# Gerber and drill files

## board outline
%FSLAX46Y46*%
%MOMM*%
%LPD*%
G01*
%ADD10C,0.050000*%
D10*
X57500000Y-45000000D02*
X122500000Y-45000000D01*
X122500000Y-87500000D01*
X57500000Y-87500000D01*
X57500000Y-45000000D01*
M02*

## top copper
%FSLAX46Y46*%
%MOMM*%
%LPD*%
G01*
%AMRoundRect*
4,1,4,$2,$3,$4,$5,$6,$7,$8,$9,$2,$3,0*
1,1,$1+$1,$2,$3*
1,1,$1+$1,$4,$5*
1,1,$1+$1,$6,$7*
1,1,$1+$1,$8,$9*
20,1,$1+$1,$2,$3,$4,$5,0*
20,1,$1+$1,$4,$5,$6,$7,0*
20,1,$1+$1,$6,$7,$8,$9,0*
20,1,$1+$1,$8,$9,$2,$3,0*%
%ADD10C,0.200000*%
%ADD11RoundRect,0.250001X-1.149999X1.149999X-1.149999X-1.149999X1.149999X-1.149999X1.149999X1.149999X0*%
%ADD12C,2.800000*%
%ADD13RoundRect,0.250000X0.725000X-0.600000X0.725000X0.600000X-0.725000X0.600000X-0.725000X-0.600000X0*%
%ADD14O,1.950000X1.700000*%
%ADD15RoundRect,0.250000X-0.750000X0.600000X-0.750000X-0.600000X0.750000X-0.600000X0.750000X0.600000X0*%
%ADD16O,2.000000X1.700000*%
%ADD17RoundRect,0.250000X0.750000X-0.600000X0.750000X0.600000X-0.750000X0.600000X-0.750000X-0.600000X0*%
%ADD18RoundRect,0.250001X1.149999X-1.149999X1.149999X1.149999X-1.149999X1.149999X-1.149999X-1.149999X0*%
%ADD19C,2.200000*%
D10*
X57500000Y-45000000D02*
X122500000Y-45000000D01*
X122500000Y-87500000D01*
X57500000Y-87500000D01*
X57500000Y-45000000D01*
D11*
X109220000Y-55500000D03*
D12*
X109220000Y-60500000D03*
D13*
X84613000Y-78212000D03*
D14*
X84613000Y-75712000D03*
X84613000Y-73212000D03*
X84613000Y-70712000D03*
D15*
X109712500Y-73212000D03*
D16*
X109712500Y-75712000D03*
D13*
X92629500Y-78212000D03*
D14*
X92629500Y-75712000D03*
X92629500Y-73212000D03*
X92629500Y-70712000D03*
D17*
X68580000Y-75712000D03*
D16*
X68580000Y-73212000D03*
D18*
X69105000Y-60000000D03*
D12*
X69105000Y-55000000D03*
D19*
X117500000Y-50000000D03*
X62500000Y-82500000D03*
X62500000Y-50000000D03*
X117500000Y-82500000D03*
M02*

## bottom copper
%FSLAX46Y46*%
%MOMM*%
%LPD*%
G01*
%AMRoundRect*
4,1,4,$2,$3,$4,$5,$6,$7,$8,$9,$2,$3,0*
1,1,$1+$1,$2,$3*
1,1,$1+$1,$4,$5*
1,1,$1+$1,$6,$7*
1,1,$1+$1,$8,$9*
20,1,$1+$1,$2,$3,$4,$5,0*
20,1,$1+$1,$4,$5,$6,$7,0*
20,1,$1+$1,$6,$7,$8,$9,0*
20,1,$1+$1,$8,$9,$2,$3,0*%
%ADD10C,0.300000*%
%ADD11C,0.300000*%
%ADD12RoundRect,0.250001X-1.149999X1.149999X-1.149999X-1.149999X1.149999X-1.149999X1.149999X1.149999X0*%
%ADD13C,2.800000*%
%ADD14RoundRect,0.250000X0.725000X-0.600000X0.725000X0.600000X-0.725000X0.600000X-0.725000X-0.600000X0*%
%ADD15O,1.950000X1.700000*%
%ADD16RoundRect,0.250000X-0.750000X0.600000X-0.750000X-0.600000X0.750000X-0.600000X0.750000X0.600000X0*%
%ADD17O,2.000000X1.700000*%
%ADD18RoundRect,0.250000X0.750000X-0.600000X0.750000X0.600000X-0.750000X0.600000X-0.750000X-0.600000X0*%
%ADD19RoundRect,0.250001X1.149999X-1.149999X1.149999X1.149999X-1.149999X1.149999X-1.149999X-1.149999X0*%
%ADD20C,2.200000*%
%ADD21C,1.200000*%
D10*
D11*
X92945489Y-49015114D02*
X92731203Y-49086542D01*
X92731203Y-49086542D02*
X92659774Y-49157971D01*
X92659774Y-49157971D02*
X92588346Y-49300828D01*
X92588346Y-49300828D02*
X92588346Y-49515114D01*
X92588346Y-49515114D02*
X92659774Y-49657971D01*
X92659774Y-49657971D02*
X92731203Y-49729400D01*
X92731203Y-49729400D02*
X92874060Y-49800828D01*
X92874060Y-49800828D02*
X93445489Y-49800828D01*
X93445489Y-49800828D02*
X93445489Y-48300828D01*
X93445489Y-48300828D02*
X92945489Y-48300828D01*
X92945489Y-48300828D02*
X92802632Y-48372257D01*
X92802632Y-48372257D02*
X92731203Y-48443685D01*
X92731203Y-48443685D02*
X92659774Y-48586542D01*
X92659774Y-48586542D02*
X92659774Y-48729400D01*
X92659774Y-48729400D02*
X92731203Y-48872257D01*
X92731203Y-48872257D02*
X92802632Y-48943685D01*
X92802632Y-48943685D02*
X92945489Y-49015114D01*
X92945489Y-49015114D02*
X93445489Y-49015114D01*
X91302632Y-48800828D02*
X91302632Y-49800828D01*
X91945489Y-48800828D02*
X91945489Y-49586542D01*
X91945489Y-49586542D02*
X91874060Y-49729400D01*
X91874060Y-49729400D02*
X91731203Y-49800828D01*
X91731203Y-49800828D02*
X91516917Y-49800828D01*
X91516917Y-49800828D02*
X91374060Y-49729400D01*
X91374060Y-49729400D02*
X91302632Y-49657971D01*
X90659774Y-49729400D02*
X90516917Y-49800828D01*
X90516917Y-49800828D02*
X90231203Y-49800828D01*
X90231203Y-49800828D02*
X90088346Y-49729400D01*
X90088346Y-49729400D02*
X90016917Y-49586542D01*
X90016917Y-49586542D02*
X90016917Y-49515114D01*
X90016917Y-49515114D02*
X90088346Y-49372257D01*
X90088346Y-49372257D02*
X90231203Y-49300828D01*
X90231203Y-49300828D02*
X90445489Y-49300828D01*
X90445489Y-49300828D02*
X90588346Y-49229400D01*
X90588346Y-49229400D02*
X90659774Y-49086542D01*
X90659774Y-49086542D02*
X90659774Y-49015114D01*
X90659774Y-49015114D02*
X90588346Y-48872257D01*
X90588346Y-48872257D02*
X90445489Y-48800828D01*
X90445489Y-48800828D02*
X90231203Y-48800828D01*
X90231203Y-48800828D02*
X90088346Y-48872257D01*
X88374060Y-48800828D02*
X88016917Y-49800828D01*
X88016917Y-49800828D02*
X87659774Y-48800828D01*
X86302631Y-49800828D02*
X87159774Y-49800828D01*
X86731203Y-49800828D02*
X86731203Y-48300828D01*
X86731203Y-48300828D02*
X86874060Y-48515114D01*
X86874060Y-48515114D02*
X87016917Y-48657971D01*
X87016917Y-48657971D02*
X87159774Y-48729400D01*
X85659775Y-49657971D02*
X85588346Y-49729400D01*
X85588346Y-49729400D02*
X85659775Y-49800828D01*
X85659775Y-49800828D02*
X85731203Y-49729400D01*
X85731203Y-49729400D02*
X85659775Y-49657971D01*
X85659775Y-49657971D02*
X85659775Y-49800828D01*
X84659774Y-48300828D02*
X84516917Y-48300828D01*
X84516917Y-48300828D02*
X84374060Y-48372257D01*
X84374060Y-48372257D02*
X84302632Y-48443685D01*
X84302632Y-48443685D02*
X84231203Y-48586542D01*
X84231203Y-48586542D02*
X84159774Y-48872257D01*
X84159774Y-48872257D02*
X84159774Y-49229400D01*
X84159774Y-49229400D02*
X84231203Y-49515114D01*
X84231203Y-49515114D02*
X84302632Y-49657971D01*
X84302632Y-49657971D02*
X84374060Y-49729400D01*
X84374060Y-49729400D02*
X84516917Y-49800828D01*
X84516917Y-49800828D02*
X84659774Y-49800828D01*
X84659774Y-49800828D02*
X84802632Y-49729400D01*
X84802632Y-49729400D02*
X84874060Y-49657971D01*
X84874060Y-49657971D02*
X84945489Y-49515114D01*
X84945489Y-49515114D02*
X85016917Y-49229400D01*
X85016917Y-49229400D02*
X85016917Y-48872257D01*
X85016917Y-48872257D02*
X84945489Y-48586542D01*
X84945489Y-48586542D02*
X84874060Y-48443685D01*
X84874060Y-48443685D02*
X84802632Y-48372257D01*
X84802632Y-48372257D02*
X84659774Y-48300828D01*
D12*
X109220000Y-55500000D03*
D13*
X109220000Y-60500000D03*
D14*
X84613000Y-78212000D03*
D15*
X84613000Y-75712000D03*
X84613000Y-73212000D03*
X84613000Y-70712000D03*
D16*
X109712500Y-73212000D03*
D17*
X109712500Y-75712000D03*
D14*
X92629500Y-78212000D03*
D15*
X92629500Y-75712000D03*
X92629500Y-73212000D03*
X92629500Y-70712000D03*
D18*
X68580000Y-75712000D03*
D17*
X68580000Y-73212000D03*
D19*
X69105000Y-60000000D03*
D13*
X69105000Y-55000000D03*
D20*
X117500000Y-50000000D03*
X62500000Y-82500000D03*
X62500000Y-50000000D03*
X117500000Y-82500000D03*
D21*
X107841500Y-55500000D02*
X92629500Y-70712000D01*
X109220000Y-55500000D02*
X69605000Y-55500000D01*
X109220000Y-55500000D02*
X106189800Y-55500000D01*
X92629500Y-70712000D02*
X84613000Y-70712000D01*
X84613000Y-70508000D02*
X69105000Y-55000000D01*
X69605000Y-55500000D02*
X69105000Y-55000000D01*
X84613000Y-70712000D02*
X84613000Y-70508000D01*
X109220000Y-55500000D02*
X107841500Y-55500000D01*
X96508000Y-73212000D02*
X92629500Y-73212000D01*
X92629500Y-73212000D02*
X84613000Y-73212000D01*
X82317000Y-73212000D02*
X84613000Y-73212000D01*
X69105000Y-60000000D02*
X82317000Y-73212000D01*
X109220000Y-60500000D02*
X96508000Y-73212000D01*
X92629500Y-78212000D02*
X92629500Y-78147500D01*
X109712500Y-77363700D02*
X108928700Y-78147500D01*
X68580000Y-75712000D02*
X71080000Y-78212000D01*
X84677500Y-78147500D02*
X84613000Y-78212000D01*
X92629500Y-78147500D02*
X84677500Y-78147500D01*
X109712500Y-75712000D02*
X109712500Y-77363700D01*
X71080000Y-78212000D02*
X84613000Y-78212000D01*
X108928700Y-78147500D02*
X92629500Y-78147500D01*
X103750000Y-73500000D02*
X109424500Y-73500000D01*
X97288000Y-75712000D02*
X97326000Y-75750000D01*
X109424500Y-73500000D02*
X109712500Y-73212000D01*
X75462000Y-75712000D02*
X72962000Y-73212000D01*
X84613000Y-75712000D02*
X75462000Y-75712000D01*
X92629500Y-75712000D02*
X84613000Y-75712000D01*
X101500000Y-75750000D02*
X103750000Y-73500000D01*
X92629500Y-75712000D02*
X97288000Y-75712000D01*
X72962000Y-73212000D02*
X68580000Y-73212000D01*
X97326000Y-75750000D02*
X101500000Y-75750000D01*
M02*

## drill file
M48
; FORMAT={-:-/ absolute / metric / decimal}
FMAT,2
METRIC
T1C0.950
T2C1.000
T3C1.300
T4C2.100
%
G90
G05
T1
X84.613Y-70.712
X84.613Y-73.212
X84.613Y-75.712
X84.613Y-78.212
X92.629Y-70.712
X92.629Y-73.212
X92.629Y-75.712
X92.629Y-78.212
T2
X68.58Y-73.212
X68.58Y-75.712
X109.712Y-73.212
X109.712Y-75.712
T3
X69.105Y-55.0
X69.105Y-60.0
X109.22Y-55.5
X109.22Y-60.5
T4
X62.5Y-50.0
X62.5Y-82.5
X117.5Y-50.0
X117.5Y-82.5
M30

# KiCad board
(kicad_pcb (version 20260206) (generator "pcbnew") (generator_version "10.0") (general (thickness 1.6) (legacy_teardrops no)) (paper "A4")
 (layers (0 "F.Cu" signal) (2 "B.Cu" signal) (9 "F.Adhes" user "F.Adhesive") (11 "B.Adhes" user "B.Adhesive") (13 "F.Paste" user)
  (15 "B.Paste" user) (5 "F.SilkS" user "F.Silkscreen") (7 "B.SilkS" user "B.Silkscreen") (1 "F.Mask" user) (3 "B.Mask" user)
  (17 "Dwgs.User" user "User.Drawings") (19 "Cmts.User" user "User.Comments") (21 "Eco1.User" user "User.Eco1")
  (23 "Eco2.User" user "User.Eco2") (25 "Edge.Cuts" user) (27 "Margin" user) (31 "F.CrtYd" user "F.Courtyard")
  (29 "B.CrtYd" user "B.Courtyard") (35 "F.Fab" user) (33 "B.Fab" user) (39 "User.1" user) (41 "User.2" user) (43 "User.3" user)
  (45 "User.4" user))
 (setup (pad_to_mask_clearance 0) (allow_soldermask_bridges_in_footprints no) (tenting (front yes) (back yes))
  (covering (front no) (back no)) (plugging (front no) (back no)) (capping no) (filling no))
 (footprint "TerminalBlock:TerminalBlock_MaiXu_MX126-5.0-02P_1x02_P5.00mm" (layer "F.Cu") (at 109.22 55.5 -90)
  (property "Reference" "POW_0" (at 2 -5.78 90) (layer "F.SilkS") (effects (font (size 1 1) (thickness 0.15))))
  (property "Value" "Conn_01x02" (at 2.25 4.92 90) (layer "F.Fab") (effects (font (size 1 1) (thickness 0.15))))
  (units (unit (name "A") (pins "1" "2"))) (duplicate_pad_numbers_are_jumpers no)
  (pad "1" thru_hole roundrect (at 0 0 270) (size 2.8 2.8) (drill 1.3) (layers "*.Cu" "*.Mask") (remove_unused_layers no)
   (roundrect_rratio 0.089286) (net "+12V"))
  (pad "2" thru_hole circle (at 5 0 270) (size 2.8 2.8) (drill 1.3) (layers "*.Cu" "*.Mask") (remove_unused_layers no) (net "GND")))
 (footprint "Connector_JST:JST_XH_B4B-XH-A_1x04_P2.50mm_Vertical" (layer "F.Cu") (at 84.613 78.212 90)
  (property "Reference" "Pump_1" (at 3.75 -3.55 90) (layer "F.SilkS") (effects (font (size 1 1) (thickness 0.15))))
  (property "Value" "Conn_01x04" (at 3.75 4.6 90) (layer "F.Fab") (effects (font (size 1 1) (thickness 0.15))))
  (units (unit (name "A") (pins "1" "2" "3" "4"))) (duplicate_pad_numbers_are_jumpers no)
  (pad "1" thru_hole roundrect (at 0 0 90) (size 1.7 1.95) (drill 0.95) (layers "*.Cu" "*.Mask") (remove_unused_layers no)
   (roundrect_rratio 0.147059) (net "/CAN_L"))
  (pad "2" thru_hole oval (at 2.5 0 90) (size 1.7 1.95) (drill 0.95) (layers "*.Cu" "*.Mask") (remove_unused_layers no) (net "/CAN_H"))
  (pad "3" thru_hole oval (at 5 0 90) (size 1.7 1.95) (drill 0.95) (layers "*.Cu" "*.Mask") (remove_unused_layers no) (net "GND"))
  (pad "4" thru_hole oval (at 7.5 0 90) (size 1.7 1.95) (drill 0.95) (layers "*.Cu" "*.Mask") (remove_unused_layers no) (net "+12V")))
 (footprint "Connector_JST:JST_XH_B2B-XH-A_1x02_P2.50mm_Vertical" (layer "F.Cu") (at 109.7125 73.212 -90)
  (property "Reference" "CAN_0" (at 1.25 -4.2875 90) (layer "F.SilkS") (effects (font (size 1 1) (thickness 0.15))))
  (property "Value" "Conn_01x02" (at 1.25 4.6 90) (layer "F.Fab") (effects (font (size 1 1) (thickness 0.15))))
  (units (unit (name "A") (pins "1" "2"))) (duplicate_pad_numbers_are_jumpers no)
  (pad "1" thru_hole roundrect (at 0 0 270) (size 1.7 2) (drill 1) (layers "*.Cu" "*.Mask") (remove_unused_layers no)
   (roundrect_rratio 0.147059) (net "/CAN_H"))
  (pad "2" thru_hole oval (at 2.5 0 270) (size 1.7 2) (drill 1) (layers "*.Cu" "*.Mask") (remove_unused_layers no) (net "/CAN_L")))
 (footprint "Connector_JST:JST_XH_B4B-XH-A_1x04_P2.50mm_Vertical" (layer "F.Cu") (at 92.6295 78.212 90)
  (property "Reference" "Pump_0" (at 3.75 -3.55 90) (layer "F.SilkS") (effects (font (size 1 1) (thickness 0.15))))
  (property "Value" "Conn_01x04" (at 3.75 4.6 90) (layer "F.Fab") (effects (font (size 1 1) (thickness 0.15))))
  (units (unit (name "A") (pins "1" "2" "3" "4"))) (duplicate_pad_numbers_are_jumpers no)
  (pad "1" thru_hole roundrect (at 0 0 90) (size 1.7 1.95) (drill 0.95) (layers "*.Cu" "*.Mask") (remove_unused_layers no)
   (roundrect_rratio 0.147059) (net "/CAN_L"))
  (pad "2" thru_hole oval (at 2.5 0 90) (size 1.7 1.95) (drill 0.95) (layers "*.Cu" "*.Mask") (remove_unused_layers no) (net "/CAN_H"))
  (pad "3" thru_hole oval (at 5 0 90) (size 1.7 1.95) (drill 0.95) (layers "*.Cu" "*.Mask") (remove_unused_layers no) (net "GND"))
  (pad "4" thru_hole oval (at 7.5 0 90) (size 1.7 1.95) (drill 0.95) (layers "*.Cu" "*.Mask") (remove_unused_layers no) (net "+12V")))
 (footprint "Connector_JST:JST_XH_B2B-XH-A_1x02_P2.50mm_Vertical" (layer "F.Cu") (at 68.58 75.712 90)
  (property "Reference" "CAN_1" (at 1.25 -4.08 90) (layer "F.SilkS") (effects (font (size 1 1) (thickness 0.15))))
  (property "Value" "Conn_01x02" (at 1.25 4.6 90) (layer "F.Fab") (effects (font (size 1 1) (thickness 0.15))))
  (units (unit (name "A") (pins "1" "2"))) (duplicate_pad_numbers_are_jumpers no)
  (pad "1" thru_hole roundrect (at 0 0 90) (size 1.7 2) (drill 1) (layers "*.Cu" "*.Mask") (remove_unused_layers no)
   (roundrect_rratio 0.147059) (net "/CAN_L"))
  (pad "2" thru_hole oval (at 2.5 0 90) (size 1.7 2) (drill 1) (layers "*.Cu" "*.Mask") (remove_unused_layers no) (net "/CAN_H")))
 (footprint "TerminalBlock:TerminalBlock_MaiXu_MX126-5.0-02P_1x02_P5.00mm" (layer "F.Cu") (at 69.105 60 90)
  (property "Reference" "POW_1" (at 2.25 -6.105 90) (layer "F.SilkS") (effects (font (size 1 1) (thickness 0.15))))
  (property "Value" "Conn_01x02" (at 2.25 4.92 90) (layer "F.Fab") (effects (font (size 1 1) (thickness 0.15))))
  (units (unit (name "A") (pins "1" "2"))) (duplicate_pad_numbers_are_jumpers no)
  (pad "1" thru_hole roundrect (at 0 0 90) (size 2.8 2.8) (drill 1.3) (layers "*.Cu" "*.Mask") (remove_unused_layers no)
   (roundrect_rratio 0.089286) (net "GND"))
  (pad "2" thru_hole circle (at 5 0 90) (size 2.8 2.8) (drill 1.3) (layers "*.Cu" "*.Mask") (remove_unused_layers no) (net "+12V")))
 (gr_rect (start 57.5 45) (end 122.5 87.5) (stroke (width 0.2) (type default)) (fill no) (layer "F.Cu"))
 (gr_rect (start 57.5 45) (end 122.5 87.5) (stroke (width 0.05) (type default)) (fill no) (layer "Edge.Cuts"))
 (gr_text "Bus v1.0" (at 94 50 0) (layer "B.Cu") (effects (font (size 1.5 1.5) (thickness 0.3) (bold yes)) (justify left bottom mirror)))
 (via (at 117.5 50) (size 2.2) (drill 2.1) (layers "F.Cu" "B.Cu") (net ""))
 (via (at 62.5 82.5) (size 2.2) (drill 2.1) (layers "F.Cu" "B.Cu") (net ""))
 (via (at 62.5 50) (size 2.2) (drill 2.1) (layers "F.Cu" "B.Cu") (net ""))
 (via (at 117.5 82.5) (size 2.2) (drill 2.1) (layers "F.Cu" "B.Cu") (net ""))
 (segment (start 107.8415 55.5) (end 92.6295 70.712) (width 1.2) (layer "B.Cu") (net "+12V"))
 (segment (start 109.22 55.5) (end 69.605 55.5) (width 1.2) (layer "B.Cu") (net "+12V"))
 (segment (start 109.22 55.5) (end 106.1898 55.5) (width 1.2) (layer "B.Cu") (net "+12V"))
 (segment (start 92.6295 70.712) (end 84.613 70.712) (width 1.2) (layer "B.Cu") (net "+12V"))
 (segment (start 84.613 70.508) (end 69.105 55) (width 1.2) (layer "B.Cu") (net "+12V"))
 (segment (start 69.605 55.5) (end 69.105 55) (width 1.2) (layer "B.Cu") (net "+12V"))
 (segment (start 84.613 70.712) (end 84.613 70.508) (width 1.2) (layer "B.Cu") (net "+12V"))
 (segment (start 109.22 55.5) (end 107.8415 55.5) (width 1.2) (layer "B.Cu") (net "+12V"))
 (segment (start 96.508 73.212) (end 92.6295 73.212) (width 1.2) (layer "B.Cu") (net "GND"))
 (segment (start 92.6295 73.212) (end 84.613 73.212) (width 1.2) (layer "B.Cu") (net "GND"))
 (segment (start 82.317 73.212) (end 84.613 73.212) (width 1.2) (layer "B.Cu") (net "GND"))
 (segment (start 69.105 60) (end 82.317 73.212) (width 1.2) (layer "B.Cu") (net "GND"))
 (segment (start 109.22 60.5) (end 96.508 73.212) (width 1.2) (layer "B.Cu") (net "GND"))
 (segment (start 92.6295 78.212) (end 92.6295 78.1475) (width 1.2) (layer "B.Cu") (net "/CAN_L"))
 (segment (start 109.7125 77.3637) (end 108.9287 78.1475) (width 1.2) (layer "B.Cu") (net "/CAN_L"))
 (segment (start 68.58 75.712) (end 71.08 78.212) (width 1.2) (layer "B.Cu") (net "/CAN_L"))
 (segment (start 84.6775 78.1475) (end 84.613 78.212) (width 1.2) (layer "B.Cu") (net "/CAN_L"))
 (segment (start 92.6295 78.1475) (end 84.6775 78.1475) (width 1.2) (layer "B.Cu") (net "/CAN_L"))
 (segment (start 109.7125 75.712) (end 109.7125 77.3637) (width 1.2) (layer "B.Cu") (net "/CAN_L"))
 (segment (start 71.08 78.212) (end 84.613 78.212) (width 1.2) (layer "B.Cu") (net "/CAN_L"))
 (segment (start 108.9287 78.1475) (end 92.6295 78.1475) (width 1.2) (layer "B.Cu") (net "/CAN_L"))
 (segment (start 103.75 73.5) (end 109.4245 73.5) (width 1.2) (layer "B.Cu") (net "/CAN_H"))
 (segment (start 97.288 75.712) (end 97.326 75.75) (width 1.2) (layer "B.Cu") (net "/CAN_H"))
 (segment (start 109.4245 73.5) (end 109.7125 73.212) (width 1.2) (layer "B.Cu") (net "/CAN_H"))
 (segment (start 75.462 75.712) (end 72.962 73.212) (width 1.2) (layer "B.Cu") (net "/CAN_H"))
 (segment (start 84.613 75.712) (end 75.462 75.712) (width 1.2) (layer "B.Cu") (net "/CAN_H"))
 (segment (start 92.6295 75.712) (end 84.613 75.712) (width 1.2) (layer "B.Cu") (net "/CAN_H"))
 (segment (start 101.5 75.75) (end 103.75 73.5) (width 1.2) (layer "B.Cu") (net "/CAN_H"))
 (segment (start 92.6295 75.712) (end 97.288 75.712) (width 1.2) (layer "B.Cu") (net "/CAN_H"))
 (segment (start 72.962 73.212) (end 68.58 73.212) (width 1.2) (layer "B.Cu") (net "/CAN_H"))
 (segment (start 97.326 75.75) (end 101.5 75.75) (width 1.2) (layer "B.Cu") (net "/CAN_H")))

